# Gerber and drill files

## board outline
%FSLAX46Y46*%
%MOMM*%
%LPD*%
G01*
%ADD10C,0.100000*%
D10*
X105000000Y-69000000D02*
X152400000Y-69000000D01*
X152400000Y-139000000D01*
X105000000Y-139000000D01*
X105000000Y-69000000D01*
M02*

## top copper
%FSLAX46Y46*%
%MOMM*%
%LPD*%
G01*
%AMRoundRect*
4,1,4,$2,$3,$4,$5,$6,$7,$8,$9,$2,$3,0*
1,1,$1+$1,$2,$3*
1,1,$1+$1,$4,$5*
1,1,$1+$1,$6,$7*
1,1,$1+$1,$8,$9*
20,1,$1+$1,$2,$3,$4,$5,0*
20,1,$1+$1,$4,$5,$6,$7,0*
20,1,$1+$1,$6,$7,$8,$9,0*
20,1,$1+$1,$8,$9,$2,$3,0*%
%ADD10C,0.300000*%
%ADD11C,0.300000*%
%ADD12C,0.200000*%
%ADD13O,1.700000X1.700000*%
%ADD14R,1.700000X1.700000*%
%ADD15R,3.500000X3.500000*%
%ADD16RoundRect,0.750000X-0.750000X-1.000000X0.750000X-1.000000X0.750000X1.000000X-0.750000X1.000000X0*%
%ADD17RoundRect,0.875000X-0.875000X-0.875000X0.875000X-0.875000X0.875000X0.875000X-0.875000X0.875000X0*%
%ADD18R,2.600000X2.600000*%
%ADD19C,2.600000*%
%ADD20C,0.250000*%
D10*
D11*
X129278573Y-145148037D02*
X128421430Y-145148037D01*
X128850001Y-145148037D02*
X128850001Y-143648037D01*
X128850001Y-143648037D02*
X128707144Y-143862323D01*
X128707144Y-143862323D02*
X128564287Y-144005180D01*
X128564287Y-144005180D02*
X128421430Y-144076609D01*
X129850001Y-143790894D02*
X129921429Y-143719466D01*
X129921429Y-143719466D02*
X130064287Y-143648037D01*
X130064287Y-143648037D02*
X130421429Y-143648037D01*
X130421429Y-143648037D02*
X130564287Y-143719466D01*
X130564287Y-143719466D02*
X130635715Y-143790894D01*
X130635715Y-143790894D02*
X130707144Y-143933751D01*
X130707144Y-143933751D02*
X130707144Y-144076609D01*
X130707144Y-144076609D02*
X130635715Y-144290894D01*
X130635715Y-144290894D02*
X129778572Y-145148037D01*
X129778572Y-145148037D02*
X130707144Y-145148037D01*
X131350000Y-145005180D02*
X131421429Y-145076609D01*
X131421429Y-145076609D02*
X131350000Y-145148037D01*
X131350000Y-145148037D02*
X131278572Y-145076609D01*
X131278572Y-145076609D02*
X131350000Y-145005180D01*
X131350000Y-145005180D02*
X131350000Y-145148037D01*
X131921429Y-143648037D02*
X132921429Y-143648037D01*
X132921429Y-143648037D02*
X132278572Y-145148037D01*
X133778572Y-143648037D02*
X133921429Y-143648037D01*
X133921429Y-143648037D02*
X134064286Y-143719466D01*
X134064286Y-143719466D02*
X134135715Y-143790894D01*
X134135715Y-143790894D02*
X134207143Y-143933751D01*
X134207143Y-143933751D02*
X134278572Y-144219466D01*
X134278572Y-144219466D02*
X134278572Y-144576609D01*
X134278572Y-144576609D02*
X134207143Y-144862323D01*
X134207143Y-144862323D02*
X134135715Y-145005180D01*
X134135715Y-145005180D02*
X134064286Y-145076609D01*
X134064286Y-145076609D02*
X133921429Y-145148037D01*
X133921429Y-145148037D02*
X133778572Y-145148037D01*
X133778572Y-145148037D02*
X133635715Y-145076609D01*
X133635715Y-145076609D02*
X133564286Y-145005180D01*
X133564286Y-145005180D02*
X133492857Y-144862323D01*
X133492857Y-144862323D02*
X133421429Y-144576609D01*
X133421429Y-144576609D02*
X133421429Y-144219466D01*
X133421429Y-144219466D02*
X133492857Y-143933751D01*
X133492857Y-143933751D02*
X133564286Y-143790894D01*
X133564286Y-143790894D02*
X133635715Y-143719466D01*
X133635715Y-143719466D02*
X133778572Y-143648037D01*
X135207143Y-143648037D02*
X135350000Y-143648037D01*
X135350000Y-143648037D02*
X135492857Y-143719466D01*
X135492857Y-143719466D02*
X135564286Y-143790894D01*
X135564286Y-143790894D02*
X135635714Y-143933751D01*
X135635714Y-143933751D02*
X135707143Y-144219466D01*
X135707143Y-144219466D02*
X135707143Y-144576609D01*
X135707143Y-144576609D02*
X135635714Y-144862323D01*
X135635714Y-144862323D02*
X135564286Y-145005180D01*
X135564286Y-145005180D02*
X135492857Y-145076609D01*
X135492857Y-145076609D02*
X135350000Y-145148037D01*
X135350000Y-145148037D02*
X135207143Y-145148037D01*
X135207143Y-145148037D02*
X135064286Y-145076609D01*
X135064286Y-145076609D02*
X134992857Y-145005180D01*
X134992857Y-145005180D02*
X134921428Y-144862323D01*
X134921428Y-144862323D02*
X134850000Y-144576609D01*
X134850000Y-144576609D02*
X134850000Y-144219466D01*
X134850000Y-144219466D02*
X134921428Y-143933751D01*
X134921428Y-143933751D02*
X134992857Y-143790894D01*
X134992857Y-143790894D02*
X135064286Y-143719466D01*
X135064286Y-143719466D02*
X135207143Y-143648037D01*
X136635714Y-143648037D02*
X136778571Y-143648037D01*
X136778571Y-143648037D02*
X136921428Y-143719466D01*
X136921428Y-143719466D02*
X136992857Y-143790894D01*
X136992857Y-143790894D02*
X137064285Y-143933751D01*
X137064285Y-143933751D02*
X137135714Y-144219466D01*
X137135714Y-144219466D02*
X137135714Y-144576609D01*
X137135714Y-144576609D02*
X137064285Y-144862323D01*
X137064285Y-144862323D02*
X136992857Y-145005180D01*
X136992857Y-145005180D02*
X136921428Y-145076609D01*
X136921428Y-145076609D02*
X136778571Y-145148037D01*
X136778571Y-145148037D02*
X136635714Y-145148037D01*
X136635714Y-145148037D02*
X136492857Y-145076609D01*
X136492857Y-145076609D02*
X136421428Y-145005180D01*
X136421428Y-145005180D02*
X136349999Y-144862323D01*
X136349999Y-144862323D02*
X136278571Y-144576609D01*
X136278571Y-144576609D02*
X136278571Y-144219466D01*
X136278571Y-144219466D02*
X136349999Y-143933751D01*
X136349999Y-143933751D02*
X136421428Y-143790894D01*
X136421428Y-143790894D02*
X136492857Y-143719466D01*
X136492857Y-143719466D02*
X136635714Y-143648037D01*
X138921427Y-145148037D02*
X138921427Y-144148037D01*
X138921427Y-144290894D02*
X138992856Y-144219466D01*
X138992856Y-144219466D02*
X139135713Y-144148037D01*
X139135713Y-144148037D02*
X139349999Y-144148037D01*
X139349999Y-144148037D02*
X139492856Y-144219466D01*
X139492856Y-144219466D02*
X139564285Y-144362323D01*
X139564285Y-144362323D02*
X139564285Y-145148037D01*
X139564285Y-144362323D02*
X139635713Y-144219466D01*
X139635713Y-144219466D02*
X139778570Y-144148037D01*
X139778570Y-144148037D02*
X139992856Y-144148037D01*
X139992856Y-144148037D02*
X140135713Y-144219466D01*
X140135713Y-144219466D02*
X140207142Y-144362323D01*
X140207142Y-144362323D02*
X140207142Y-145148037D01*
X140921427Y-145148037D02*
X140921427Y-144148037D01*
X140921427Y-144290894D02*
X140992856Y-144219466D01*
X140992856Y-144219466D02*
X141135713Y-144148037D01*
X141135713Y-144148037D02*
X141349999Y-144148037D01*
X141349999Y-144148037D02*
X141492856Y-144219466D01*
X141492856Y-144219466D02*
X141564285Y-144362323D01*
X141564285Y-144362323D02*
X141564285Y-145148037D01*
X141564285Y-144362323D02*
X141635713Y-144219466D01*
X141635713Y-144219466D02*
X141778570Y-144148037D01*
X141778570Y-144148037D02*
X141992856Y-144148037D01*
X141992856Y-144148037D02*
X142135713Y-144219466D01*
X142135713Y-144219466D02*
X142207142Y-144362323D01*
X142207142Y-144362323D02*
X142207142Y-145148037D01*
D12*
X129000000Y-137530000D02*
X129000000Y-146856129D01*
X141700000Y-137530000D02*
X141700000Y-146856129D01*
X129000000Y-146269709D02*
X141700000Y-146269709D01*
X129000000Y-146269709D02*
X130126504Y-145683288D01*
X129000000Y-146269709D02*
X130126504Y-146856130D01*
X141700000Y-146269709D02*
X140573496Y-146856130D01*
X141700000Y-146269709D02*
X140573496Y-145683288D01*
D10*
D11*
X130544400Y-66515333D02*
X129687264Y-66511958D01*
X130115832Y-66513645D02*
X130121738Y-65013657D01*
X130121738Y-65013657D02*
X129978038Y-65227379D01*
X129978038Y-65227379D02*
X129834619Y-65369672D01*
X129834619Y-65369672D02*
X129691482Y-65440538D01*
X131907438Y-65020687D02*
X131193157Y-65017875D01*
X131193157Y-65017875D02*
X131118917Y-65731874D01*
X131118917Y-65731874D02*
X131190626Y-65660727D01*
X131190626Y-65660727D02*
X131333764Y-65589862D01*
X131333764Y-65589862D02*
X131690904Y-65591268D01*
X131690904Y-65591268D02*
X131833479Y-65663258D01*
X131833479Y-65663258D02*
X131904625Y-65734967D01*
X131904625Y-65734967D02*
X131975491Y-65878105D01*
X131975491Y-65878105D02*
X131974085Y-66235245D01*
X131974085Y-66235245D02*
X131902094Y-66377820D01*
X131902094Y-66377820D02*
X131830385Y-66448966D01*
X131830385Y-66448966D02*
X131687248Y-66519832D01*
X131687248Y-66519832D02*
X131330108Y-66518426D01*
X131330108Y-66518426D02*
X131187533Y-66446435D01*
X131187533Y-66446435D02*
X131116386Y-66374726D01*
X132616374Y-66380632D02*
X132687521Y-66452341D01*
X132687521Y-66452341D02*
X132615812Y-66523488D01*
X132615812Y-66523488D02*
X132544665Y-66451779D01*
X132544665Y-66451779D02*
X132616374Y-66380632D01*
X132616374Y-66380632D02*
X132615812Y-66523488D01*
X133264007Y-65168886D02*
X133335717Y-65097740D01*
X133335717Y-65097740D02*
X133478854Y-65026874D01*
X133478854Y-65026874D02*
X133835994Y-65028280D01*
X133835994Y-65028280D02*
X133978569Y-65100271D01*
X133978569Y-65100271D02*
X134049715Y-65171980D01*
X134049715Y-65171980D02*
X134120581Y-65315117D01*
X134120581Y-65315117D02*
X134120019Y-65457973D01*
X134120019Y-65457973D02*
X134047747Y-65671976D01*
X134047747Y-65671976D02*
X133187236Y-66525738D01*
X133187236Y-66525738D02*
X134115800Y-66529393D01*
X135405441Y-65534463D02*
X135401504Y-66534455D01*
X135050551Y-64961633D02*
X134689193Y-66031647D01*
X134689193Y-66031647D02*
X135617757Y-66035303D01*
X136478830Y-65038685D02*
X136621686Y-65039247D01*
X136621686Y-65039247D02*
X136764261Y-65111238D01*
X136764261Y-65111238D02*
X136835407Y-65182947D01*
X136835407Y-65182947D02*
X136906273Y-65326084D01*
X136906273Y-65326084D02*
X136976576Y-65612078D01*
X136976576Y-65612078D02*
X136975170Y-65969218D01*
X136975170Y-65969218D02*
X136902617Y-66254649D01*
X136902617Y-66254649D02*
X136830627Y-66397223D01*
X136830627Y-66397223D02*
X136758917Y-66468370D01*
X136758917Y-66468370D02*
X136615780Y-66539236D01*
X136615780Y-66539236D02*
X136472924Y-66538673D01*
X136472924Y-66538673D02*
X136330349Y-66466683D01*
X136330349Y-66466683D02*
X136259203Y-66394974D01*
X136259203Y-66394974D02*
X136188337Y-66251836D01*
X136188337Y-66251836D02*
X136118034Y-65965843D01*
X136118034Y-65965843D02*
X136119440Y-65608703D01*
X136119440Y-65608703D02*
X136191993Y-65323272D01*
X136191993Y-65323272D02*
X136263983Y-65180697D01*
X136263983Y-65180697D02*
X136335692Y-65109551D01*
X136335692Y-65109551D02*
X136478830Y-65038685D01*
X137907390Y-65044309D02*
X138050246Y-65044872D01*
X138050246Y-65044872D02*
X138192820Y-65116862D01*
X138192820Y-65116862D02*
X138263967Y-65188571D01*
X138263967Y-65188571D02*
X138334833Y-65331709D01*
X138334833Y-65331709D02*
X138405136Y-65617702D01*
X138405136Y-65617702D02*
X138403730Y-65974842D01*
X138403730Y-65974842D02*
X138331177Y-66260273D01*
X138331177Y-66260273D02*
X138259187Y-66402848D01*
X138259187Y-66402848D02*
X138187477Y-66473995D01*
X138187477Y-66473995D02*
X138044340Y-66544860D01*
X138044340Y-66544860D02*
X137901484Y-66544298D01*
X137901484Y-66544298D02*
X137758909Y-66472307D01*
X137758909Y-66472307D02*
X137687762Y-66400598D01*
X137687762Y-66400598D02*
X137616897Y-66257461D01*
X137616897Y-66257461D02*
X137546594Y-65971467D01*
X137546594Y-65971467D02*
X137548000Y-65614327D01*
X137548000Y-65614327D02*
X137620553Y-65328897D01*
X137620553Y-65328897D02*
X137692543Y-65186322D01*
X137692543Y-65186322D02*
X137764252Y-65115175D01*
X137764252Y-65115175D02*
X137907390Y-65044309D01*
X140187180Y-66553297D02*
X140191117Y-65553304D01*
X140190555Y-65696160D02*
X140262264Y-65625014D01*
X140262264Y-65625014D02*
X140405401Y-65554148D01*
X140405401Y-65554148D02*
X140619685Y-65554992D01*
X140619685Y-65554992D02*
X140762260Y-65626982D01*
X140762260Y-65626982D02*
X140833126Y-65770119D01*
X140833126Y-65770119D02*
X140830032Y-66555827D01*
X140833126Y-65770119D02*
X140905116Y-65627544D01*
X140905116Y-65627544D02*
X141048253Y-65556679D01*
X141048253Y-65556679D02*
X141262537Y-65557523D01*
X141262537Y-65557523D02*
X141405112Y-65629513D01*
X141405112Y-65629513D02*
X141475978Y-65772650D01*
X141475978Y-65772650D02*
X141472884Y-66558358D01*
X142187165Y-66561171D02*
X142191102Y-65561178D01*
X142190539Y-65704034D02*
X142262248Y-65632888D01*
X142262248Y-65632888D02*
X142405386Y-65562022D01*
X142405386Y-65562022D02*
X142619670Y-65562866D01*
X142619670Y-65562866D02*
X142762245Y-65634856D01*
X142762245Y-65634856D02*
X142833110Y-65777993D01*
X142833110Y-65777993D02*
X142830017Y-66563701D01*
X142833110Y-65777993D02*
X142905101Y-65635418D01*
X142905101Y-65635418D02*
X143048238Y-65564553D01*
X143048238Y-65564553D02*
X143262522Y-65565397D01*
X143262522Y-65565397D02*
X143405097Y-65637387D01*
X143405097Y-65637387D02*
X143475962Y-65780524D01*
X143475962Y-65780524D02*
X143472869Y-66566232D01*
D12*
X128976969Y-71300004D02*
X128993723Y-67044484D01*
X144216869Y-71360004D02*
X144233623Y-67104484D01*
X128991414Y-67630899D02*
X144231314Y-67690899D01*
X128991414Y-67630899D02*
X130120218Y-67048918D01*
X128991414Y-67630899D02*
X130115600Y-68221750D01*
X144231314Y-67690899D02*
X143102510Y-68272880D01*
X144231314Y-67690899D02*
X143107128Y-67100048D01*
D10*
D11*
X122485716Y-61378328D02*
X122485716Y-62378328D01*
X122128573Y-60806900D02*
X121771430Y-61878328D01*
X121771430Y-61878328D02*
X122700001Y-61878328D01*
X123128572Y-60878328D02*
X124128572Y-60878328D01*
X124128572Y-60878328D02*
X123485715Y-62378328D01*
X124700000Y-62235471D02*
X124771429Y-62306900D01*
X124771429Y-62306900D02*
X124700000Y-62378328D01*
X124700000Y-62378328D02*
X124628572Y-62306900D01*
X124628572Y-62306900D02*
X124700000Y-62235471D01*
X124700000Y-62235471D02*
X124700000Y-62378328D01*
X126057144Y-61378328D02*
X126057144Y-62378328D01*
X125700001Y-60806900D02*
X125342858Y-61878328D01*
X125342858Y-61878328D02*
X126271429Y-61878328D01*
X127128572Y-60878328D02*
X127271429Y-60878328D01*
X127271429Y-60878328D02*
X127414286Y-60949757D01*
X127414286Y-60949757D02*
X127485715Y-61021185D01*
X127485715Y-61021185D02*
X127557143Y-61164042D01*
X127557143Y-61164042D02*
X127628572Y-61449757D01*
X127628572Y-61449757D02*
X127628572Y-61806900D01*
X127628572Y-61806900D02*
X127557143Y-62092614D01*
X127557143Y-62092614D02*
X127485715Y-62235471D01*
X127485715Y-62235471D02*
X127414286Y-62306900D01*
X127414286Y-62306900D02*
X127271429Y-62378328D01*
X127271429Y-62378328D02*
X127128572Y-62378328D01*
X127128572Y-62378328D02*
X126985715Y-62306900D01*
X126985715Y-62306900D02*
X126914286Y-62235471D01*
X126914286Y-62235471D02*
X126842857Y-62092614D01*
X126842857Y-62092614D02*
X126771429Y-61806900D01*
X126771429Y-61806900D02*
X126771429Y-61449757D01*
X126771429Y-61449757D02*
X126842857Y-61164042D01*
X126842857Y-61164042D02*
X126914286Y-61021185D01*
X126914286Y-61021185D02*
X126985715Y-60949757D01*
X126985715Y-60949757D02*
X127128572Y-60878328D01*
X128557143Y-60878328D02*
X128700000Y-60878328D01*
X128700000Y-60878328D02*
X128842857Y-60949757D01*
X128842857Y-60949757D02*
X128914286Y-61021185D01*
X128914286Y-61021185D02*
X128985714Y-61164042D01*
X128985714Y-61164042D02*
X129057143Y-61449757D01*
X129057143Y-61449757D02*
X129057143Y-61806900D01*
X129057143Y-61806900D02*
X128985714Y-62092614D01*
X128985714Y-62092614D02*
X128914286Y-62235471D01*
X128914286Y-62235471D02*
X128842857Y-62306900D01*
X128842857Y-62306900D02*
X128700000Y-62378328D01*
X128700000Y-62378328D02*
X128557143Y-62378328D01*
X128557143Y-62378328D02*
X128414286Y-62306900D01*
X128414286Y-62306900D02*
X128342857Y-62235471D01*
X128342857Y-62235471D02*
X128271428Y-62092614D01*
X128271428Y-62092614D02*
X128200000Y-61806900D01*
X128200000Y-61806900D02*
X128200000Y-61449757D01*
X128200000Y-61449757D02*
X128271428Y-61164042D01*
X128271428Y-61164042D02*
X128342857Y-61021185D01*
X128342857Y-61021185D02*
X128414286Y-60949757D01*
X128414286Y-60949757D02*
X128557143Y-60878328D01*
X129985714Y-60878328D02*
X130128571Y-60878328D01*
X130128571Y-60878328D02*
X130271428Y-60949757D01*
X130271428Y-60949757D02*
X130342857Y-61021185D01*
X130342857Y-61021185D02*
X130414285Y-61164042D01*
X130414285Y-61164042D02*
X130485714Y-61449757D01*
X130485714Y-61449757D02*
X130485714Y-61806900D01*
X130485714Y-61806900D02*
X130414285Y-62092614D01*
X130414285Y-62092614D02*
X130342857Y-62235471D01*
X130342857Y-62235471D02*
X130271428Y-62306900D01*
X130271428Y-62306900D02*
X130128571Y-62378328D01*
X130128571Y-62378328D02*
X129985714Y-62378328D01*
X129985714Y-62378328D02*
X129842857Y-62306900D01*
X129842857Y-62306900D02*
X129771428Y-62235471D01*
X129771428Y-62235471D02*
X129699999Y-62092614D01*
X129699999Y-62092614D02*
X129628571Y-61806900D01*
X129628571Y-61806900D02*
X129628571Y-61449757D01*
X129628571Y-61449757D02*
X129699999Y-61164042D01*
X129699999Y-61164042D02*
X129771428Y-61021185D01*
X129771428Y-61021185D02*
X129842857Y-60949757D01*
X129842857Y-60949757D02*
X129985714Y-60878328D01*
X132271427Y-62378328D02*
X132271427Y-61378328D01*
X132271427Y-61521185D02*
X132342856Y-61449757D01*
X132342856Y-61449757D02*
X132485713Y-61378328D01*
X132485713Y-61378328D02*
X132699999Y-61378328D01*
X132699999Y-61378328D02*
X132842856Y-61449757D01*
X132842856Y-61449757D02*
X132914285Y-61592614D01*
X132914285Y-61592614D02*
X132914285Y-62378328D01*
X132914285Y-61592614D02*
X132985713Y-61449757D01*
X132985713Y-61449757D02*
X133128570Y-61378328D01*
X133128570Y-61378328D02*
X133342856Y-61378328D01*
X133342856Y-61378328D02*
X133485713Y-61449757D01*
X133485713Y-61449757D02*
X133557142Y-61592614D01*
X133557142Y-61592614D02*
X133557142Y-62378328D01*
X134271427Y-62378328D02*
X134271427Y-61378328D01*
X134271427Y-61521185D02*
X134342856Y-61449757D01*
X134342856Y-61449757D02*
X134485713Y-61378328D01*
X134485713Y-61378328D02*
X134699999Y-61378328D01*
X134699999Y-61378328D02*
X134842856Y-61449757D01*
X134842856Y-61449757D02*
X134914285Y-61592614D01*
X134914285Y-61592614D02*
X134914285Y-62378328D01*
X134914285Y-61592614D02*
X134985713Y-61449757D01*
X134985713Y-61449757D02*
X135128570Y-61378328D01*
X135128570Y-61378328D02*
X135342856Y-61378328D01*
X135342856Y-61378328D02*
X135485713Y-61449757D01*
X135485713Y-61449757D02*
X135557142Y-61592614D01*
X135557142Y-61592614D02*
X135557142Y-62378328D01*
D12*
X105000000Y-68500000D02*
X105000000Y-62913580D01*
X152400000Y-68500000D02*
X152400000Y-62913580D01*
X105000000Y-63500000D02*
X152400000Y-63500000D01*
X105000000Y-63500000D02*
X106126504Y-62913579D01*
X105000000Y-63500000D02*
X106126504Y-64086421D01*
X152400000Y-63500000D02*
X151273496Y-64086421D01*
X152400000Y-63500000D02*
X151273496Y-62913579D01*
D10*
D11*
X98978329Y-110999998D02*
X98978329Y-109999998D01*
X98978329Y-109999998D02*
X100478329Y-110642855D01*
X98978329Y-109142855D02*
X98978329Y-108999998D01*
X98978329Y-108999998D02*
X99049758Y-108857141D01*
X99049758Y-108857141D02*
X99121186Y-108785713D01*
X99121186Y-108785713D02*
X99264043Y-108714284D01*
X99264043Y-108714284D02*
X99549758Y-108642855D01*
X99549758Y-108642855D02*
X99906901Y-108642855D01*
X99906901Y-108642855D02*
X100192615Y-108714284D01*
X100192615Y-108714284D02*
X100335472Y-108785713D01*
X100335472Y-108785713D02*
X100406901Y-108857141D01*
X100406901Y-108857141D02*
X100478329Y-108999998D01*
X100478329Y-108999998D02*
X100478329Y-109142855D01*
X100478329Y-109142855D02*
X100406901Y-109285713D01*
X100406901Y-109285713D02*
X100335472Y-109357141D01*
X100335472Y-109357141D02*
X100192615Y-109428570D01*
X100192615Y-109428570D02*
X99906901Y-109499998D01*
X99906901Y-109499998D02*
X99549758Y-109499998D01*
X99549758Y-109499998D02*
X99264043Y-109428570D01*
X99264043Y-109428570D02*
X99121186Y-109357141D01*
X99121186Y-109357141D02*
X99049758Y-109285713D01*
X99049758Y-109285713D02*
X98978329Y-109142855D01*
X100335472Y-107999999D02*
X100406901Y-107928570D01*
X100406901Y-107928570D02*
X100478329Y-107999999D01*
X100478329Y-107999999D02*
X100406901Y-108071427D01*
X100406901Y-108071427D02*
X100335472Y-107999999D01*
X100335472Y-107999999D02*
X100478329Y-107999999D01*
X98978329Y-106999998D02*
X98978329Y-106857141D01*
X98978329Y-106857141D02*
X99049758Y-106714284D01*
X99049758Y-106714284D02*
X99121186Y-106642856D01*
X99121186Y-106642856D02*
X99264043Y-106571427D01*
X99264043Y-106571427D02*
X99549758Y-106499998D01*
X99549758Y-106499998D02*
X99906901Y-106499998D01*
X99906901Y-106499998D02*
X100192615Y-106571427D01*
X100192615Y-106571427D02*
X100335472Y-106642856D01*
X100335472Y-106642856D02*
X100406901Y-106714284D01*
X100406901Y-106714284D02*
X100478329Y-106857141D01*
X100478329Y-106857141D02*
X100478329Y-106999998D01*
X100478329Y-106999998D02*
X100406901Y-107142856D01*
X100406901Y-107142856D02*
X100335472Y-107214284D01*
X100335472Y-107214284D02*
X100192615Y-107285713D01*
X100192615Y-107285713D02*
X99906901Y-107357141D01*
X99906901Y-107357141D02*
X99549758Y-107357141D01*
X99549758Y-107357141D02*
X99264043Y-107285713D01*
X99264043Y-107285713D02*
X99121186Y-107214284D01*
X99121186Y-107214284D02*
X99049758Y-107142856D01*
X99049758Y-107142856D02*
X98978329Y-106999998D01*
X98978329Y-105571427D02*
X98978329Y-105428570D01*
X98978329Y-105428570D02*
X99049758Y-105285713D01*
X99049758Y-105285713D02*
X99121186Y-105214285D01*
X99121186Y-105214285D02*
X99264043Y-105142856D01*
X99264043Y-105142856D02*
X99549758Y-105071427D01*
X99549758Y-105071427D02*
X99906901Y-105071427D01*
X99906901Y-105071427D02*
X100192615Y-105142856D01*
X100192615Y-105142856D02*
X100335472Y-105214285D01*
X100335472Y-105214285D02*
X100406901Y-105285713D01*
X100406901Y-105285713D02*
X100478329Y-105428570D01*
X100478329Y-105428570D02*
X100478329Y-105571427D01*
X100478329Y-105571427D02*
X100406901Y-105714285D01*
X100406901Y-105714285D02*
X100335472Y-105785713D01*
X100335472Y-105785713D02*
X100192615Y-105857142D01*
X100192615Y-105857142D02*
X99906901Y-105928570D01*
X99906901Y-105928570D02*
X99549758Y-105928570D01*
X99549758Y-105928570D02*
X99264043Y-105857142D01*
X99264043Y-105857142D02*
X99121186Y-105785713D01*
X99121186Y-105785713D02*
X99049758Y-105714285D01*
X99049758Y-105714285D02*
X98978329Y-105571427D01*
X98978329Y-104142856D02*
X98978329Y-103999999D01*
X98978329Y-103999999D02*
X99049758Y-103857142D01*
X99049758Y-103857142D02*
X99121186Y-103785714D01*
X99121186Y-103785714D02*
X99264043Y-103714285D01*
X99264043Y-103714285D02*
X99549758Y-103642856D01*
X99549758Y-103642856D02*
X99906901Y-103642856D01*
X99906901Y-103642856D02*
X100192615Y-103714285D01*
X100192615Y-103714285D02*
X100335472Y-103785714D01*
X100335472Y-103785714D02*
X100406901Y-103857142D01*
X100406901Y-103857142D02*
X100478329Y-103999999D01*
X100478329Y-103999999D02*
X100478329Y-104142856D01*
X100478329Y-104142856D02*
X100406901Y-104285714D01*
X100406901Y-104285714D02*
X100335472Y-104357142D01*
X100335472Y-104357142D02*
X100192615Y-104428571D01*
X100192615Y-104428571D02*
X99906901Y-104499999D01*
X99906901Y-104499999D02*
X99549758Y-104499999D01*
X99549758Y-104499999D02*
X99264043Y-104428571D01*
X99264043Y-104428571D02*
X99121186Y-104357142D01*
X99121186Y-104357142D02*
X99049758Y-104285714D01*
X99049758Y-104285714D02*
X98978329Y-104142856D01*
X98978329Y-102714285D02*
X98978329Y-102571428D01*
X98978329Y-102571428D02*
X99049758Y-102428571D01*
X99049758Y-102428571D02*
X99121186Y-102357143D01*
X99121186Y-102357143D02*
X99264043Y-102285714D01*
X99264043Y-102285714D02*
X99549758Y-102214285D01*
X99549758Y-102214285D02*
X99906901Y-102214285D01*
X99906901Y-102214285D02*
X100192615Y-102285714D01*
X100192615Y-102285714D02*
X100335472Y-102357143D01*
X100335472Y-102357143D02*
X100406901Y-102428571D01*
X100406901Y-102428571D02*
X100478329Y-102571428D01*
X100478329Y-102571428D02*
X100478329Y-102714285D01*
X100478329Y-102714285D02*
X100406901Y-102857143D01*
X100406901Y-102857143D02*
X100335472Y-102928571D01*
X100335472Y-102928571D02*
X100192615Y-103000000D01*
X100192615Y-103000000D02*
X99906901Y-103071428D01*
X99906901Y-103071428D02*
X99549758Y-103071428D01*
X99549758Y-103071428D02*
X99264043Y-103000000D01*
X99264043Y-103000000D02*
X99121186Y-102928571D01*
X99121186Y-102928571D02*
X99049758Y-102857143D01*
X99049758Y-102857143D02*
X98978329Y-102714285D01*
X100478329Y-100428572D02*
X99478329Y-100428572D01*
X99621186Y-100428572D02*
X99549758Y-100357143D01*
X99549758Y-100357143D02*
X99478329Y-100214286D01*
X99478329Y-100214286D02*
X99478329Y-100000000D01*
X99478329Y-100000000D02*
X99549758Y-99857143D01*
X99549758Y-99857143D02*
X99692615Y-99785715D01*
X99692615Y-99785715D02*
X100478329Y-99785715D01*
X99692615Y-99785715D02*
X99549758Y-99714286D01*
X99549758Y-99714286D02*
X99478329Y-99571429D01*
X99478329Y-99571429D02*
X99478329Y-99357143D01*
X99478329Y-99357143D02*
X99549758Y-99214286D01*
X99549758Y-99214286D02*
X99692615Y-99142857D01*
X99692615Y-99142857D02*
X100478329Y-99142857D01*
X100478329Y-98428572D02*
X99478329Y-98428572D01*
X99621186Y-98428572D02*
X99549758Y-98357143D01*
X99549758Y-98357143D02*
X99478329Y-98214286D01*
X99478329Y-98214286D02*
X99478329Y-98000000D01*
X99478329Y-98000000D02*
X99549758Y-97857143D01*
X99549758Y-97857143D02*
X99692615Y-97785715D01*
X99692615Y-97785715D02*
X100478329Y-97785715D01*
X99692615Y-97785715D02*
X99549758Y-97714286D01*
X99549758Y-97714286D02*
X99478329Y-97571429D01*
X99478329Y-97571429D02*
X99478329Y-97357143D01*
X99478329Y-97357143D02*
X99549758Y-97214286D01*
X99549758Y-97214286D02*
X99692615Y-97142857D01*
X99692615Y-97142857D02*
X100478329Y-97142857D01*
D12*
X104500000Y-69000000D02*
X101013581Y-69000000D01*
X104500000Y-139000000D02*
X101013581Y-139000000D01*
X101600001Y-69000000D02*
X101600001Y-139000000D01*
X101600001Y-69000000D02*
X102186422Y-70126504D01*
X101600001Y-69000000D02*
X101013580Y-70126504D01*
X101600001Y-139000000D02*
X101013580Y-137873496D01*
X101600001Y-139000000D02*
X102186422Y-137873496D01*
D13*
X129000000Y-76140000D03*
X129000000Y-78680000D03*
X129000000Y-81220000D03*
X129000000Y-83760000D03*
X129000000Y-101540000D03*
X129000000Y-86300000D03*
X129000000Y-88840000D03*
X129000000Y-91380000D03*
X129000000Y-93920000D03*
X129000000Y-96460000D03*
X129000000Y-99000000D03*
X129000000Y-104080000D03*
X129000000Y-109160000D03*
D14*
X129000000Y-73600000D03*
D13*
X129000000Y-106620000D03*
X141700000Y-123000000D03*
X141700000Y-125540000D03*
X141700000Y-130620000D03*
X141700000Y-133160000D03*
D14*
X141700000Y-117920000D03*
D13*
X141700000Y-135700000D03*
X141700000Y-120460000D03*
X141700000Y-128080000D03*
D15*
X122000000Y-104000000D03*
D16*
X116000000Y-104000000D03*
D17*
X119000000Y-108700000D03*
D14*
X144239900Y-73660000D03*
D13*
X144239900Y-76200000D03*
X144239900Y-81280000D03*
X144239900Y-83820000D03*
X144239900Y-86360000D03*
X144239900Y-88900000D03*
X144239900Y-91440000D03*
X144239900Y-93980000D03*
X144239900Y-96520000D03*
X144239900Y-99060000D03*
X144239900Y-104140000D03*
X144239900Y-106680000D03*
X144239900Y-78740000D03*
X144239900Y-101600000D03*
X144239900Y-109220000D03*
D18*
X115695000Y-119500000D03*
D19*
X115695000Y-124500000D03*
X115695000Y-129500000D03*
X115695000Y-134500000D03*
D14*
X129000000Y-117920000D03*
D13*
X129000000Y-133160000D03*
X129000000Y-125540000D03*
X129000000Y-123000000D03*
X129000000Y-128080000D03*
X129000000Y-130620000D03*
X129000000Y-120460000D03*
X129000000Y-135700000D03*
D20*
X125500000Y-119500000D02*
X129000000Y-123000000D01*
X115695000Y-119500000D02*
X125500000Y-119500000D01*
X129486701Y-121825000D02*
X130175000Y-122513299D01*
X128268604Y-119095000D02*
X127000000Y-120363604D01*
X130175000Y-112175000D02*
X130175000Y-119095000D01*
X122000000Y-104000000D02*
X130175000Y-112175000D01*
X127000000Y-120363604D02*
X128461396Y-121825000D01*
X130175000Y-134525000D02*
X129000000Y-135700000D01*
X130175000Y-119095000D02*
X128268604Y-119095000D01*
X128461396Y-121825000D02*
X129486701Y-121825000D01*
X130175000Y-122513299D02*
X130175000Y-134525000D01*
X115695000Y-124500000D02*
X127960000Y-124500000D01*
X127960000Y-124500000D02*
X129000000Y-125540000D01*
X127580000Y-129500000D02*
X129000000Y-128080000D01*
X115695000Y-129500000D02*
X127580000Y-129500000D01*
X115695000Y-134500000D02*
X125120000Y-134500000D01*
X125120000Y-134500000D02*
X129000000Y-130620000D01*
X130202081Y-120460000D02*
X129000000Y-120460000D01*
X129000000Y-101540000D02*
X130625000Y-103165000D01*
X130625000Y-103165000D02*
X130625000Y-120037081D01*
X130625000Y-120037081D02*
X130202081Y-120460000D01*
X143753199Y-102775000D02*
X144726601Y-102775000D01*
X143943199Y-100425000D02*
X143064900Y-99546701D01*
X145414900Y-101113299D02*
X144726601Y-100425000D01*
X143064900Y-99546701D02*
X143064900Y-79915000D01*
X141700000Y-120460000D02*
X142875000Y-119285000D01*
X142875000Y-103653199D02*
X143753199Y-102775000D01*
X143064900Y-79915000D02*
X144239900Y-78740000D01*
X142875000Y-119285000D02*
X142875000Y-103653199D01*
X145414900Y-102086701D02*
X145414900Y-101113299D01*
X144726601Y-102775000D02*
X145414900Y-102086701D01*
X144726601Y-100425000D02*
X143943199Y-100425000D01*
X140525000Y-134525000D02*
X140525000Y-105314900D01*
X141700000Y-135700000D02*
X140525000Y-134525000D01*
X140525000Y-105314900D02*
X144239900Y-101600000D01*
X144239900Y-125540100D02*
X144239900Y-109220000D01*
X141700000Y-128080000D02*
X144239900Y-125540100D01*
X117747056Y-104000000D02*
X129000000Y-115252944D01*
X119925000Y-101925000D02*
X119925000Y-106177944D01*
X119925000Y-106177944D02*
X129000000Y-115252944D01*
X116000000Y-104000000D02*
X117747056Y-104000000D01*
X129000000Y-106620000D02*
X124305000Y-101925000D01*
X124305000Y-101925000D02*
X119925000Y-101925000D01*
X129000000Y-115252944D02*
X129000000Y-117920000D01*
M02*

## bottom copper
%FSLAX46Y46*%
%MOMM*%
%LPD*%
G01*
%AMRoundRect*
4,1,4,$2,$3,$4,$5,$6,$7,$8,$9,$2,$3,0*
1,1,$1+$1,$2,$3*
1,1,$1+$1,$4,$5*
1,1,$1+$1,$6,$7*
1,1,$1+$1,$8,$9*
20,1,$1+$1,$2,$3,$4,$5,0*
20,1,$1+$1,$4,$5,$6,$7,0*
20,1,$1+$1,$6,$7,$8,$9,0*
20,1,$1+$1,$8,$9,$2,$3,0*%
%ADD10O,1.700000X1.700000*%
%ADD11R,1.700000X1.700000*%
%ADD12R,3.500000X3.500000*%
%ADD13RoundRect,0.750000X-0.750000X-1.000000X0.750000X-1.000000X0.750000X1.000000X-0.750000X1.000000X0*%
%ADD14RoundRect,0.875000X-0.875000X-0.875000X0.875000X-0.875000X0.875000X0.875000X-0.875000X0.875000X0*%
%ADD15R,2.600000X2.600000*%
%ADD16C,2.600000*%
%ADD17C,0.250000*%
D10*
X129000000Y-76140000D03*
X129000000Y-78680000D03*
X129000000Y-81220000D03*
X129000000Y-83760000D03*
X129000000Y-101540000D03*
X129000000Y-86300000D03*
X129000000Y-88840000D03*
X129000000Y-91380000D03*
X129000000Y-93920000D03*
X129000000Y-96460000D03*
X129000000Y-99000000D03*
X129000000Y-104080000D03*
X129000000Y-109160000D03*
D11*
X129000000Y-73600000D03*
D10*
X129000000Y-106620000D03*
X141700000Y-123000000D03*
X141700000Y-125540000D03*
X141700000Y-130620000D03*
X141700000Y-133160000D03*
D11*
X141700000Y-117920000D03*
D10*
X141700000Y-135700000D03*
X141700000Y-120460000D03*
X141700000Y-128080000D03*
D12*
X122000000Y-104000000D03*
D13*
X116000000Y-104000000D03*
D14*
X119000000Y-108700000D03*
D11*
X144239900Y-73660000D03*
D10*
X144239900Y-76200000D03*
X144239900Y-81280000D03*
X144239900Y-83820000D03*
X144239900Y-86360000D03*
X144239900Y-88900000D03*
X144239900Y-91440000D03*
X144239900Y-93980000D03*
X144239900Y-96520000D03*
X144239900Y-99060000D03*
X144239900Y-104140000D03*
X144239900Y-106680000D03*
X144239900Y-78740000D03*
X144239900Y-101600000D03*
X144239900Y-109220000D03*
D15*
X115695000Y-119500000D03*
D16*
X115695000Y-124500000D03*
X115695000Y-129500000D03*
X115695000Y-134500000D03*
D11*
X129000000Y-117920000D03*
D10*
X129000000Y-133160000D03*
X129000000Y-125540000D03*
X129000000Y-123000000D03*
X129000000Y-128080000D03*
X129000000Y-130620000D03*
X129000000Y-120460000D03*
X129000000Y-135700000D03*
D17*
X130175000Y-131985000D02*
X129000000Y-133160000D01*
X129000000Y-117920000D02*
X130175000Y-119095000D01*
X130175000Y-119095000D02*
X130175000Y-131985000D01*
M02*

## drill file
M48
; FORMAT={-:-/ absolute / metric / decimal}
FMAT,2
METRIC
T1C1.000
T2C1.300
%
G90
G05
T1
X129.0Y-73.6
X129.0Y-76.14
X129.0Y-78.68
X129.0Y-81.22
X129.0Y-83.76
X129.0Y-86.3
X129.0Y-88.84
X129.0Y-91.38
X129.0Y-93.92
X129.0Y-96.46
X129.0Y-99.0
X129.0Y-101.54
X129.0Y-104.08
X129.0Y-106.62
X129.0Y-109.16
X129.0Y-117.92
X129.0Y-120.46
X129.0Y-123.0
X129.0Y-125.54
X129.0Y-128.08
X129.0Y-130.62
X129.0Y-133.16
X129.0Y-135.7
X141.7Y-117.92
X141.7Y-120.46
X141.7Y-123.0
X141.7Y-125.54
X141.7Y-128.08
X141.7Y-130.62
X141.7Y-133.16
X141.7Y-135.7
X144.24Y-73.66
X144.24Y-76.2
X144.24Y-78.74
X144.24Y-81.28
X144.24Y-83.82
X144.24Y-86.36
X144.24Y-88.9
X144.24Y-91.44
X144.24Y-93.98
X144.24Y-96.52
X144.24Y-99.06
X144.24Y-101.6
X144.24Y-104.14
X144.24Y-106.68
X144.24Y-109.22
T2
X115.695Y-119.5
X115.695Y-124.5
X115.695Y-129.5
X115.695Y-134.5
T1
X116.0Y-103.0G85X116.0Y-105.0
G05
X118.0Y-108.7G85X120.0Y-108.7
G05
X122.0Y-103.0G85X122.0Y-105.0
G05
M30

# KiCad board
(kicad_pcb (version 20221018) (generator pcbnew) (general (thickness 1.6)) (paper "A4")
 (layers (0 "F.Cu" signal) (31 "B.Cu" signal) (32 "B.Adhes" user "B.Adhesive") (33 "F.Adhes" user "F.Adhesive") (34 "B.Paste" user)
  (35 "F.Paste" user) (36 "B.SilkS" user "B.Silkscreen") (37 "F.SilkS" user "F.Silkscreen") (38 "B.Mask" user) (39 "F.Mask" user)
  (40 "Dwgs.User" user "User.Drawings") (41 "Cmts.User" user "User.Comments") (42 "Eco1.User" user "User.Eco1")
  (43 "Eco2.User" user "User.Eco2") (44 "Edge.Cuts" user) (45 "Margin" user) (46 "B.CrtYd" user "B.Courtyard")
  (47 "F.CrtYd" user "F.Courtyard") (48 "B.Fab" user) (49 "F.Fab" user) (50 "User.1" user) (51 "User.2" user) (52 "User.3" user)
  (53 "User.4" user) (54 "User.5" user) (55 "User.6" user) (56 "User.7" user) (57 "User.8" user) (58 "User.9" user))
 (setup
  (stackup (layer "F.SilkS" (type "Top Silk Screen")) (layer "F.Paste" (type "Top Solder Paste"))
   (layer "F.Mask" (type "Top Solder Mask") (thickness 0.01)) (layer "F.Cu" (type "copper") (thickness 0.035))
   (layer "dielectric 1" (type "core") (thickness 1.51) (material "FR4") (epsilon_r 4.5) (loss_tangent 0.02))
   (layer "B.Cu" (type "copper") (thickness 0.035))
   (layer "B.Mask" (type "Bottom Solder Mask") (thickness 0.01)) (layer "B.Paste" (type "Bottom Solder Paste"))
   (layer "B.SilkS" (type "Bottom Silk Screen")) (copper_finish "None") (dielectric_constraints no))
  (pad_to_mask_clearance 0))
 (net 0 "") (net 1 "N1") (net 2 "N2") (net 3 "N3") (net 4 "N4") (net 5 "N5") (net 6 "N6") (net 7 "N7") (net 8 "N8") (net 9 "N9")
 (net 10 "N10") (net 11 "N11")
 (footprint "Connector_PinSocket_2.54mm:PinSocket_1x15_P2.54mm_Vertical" (layer "F.Cu") (at 129 73.6)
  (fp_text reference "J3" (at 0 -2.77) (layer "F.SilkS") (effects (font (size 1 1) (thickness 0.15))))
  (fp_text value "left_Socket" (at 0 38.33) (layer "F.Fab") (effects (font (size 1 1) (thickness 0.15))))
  (pad "2" thru_hole oval (at 0 2.54) (size 1.7 1.7) (drill 1) (layers "*.Cu" "*.Mask"))
  (pad "3" thru_hole oval (at 0 5.08) (size 1.7 1.7) (drill 1) (layers "*.Cu" "*.Mask"))
  (pad "4" thru_hole oval (at 0 7.62) (size 1.7 1.7) (drill 1) (layers "*.Cu" "*.Mask"))
  (pad "5" thru_hole oval (at 0 10.16) (size 1.7 1.7) (drill 1) (layers "*.Cu" "*.Mask"))
  (pad "5V" thru_hole oval (at 0 27.94) (size 1.7 1.7) (drill 1) (layers "*.Cu" "*.Mask") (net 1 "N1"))
  (pad "6" thru_hole oval (at 0 12.7) (size 1.7 1.7) (drill 1) (layers "*.Cu" "*.Mask"))
  (pad "7" thru_hole oval (at 0 15.24) (size 1.7 1.7) (drill 1) (layers "*.Cu" "*.Mask"))
  (pad "8" thru_hole oval (at 0 17.78) (size 1.7 1.7) (drill 1) (layers "*.Cu" "*.Mask"))
  (pad "9" thru_hole oval (at 0 20.32) (size 1.7 1.7) (drill 1) (layers "*.Cu" "*.Mask"))
  (pad "10" thru_hole oval (at 0 22.86) (size 1.7 1.7) (drill 1) (layers "*.Cu" "*.Mask"))
  (pad "11" thru_hole oval (at 0 25.4) (size 1.7 1.7) (drill 1) (layers "*.Cu" "*.Mask"))
  (pad "13" thru_hole oval (at 0 30.48) (size 1.7 1.7) (drill 1) (layers "*.Cu" "*.Mask"))
  (pad "15" thru_hole oval (at 0 35.56) (size 1.7 1.7) (drill 1) (layers "*.Cu" "*.Mask"))
  (pad "D12" thru_hole rect (at 0 0) (size 1.7 1.7) (drill 1) (layers "*.Cu" "*.Mask"))
  (pad "GND" thru_hole oval (at 0 33.02) (size 1.7 1.7) (drill 1) (layers "*.Cu" "*.Mask") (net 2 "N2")))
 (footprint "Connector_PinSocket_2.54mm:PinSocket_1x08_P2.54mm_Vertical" (layer "F.Cu") (at 141.7 117.92)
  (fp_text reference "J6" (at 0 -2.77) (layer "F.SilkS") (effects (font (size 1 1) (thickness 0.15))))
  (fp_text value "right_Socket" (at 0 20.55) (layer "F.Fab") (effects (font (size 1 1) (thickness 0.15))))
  (pad "3" thru_hole oval (at 0 5.08) (size 1.7 1.7) (drill 1) (layers "*.Cu" "*.Mask"))
  (pad "4" thru_hole oval (at 0 7.62) (size 1.7 1.7) (drill 1) (layers "*.Cu" "*.Mask"))
  (pad "6" thru_hole oval (at 0 12.7) (size 1.7 1.7) (drill 1) (layers "*.Cu" "*.Mask"))
  (pad "7" thru_hole oval (at 0 15.24) (size 1.7 1.7) (drill 1) (layers "*.Cu" "*.Mask"))
  (pad "Dir" thru_hole rect (at 0 0) (size 1.7 1.7) (drill 1) (layers "*.Cu" "*.Mask") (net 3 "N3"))
  (pad "EN" thru_hole oval (at 0 17.78) (size 1.7 1.7) (drill 1) (layers "*.Cu" "*.Mask") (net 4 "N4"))
  (pad "Step" thru_hole oval (at 0 2.54) (size 1.7 1.7) (drill 1) (layers "*.Cu" "*.Mask") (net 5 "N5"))
  (pad "UART" thru_hole oval (at 0 10.16) (size 1.7 1.7) (drill 1) (layers "*.Cu" "*.Mask") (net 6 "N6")))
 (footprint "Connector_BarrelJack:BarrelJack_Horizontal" (layer "F.Cu") (at 122 104)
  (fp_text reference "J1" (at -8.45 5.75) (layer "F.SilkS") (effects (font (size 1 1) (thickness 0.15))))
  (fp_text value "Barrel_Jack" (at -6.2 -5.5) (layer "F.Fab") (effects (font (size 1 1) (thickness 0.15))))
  (pad "1" thru_hole rect (at 0 0) (size 3.5 3.5) (drill oval 1 3) (layers "*.Cu" "*.Mask") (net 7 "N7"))
  (pad "2" thru_hole roundrect (at -6 0) (size 3 3.5) (drill oval 1 3) (layers "*.Cu" "*.Mask") (roundrect_rratio 0.25) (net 2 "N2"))
  (pad "3" thru_hole roundrect (at -3 4.7) (size 3.5 3.5) (drill oval 3 1) (layers "*.Cu" "*.Mask") (roundrect_rratio 0.25)))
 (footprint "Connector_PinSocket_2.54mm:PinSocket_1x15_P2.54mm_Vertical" (layer "F.Cu") (at 144.2399 73.66)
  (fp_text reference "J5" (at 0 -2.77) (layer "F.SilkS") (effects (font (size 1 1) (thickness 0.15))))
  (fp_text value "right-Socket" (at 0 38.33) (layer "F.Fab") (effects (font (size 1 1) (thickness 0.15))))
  (pad "1" thru_hole rect (at 0 0) (size 1.7 1.7) (drill 1) (layers "*.Cu" "*.Mask"))
  (pad "2" thru_hole oval (at 0 2.54) (size 1.7 1.7) (drill 1) (layers "*.Cu" "*.Mask"))
  (pad "4" thru_hole oval (at 0 7.62) (size 1.7 1.7) (drill 1) (layers "*.Cu" "*.Mask"))
  (pad "5" thru_hole oval (at 0 10.16) (size 1.7 1.7) (drill 1) (layers "*.Cu" "*.Mask"))
  (pad "6" thru_hole oval (at 0 12.7) (size 1.7 1.7) (drill 1) (layers "*.Cu" "*.Mask"))
  (pad "7" thru_hole oval (at 0 15.24) (size 1.7 1.7) (drill 1) (layers "*.Cu" "*.Mask"))
  (pad "8" thru_hole oval (at 0 17.78) (size 1.7 1.7) (drill 1) (layers "*.Cu" "*.Mask"))
  (pad "9" thru_hole oval (at 0 20.32) (size 1.7 1.7) (drill 1) (layers "*.Cu" "*.Mask"))
  (pad "10" thru_hole oval (at 0 22.86) (size 1.7 1.7) (drill 1) (layers "*.Cu" "*.Mask"))
  (pad "11" thru_hole oval (at 0 25.4) (size 1.7 1.7) (drill 1) (layers "*.Cu" "*.Mask"))
  (pad "13" thru_hole oval (at 0 30.48) (size 1.7 1.7) (drill 1) (layers "*.Cu" "*.Mask"))
  (pad "14" thru_hole oval (at 0 33.02) (size 1.7 1.7) (drill 1) (layers "*.Cu" "*.Mask"))
  (pad "D10" thru_hole oval (at 0 5.08) (size 1.7 1.7) (drill 1) (layers "*.Cu" "*.Mask") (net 5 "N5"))
  (pad "GND" thru_hole oval (at 0 27.94) (size 1.7 1.7) (drill 1) (layers "*.Cu" "*.Mask") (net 4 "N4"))
  (pad "TX1" thru_hole oval (at 0 35.56) (size 1.7 1.7) (drill 1) (layers "*.Cu" "*.Mask") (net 6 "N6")))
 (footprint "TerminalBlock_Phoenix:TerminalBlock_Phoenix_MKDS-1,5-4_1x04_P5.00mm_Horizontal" (layer "F.Cu") (at 115.695 119.5 -90)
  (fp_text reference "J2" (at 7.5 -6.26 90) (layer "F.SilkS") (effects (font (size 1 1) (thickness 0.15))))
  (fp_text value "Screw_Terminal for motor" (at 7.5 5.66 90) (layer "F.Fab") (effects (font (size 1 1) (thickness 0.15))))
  (pad "1" thru_hole rect (at 0 0 270) (size 2.6 2.6) (drill 1.3) (layers "*.Cu" "*.Mask") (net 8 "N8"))
  (pad "2" thru_hole circle (at 5 0 270) (size 2.6 2.6) (drill 1.3) (layers "*.Cu" "*.Mask") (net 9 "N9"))
  (pad "3" thru_hole circle (at 10 0 270) (size 2.6 2.6) (drill 1.3) (layers "*.Cu" "*.Mask") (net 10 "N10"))
  (pad "4" thru_hole circle (at 15 0 270) (size 2.6 2.6) (drill 1.3) (layers "*.Cu" "*.Mask") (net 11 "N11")))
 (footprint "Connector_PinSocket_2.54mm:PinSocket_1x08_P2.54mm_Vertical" (layer "F.Cu") (at 129 117.92)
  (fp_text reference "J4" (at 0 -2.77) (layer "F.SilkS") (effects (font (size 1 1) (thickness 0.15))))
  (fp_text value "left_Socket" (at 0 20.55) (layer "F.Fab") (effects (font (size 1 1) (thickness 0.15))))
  (pad "GND" thru_hole rect (at 0 0) (size 1.7 1.7) (drill 1) (layers "*.Cu" "*.Mask") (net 2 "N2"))
  (pad "GND" thru_hole oval (at 0 15.24) (size 1.7 1.7) (drill 1) (layers "*.Cu" "*.Mask") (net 2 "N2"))
  (pad "M1A" thru_hole oval (at 0 7.62) (size 1.7 1.7) (drill 1) (layers "*.Cu" "*.Mask") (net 9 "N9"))
  (pad "M1B" thru_hole oval (at 0 5.08) (size 1.7 1.7) (drill 1) (layers "*.Cu" "*.Mask") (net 8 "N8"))
  (pad "M2A" thru_hole oval (at 0 10.16) (size 1.7 1.7) (drill 1) (layers "*.Cu" "*.Mask") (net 10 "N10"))
  (pad "M2B" thru_hole oval (at 0 12.7) (size 1.7 1.7) (drill 1) (layers "*.Cu" "*.Mask") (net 11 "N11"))
  (pad "VIO" thru_hole oval (at 0 2.54) (size 1.7 1.7) (drill 1) (layers "*.Cu" "*.Mask") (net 1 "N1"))
  (pad "VM" thru_hole oval (at 0 17.78) (size 1.7 1.7) (drill 1) (layers "*.Cu" "*.Mask") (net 7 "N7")))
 (gr_rect (start 105 69) (end 152.4 139) (stroke (width 0.1) (type default)) (fill none) (layer "Edge.Cuts"))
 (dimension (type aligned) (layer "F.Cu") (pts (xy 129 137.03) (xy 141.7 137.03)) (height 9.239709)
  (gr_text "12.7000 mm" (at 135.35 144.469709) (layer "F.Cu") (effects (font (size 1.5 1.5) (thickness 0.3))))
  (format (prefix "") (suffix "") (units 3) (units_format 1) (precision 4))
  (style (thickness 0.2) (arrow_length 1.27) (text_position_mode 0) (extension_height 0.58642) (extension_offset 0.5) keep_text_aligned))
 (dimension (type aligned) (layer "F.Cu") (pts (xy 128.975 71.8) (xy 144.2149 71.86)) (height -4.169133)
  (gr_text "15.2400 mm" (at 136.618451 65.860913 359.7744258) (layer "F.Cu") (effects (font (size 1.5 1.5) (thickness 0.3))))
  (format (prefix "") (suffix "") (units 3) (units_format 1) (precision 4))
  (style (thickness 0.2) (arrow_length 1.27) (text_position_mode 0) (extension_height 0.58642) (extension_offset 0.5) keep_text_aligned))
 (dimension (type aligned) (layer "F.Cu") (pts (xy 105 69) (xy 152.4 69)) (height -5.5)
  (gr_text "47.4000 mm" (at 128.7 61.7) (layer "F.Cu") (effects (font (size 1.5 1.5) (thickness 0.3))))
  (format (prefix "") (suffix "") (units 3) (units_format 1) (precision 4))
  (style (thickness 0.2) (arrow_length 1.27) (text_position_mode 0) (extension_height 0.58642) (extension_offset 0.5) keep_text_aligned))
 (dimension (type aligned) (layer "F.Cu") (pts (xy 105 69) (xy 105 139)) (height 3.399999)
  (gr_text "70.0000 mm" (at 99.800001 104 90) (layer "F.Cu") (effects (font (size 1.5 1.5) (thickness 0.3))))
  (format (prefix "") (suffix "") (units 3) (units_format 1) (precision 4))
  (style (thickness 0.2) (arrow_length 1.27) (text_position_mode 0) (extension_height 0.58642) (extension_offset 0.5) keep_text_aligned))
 (segment (start 125.5 119.5) (end 129 123) (width 0.25) (layer "F.Cu") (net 8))
 (segment (start 115.695 119.5) (end 125.5 119.5) (width 0.25) (layer "F.Cu") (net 8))
 (segment (start 129.486701 121.825) (end 130.175 122.513299) (width 0.25) (layer "F.Cu") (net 7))
 (segment (start 128.268604 119.095) (end 127 120.363604) (width 0.25) (layer "F.Cu") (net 7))
 (segment (start 130.175 112.175) (end 130.175 119.095) (width 0.25) (layer "F.Cu") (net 7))
 (segment (start 122 104) (end 130.175 112.175) (width 0.25) (layer "F.Cu") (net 7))
 (segment (start 127 120.363604) (end 128.461396 121.825) (width 0.25) (layer "F.Cu") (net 7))
 (segment (start 130.175 134.525) (end 129 135.7) (width 0.25) (layer "F.Cu") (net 7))
 (segment (start 130.175 119.095) (end 128.268604 119.095) (width 0.25) (layer "F.Cu") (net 7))
 (segment (start 128.461396 121.825) (end 129.486701 121.825) (width 0.25) (layer "F.Cu") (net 7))
 (segment (start 130.175 122.513299) (end 130.175 134.525) (width 0.25) (layer "F.Cu") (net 7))
 (segment (start 115.695 124.5) (end 127.96 124.5) (width 0.25) (layer "F.Cu") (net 9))
 (segment (start 127.96 124.5) (end 129 125.54) (width 0.25) (layer "F.Cu") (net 9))
 (segment (start 127.58 129.5) (end 129 128.08) (width 0.25) (layer "F.Cu") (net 10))
 (segment (start 115.695 129.5) (end 127.58 129.5) (width 0.25) (layer "F.Cu") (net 10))
 (segment (start 115.695 134.5) (end 125.12 134.5) (width 0.25) (layer "F.Cu") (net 11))
 (segment (start 125.12 134.5) (end 129 130.62) (width 0.25) (layer "F.Cu") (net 11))
 (segment (start 130.202081 120.46) (end 129 120.46) (width 0.25) (layer "F.Cu") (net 1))
 (segment (start 129 101.54) (end 130.625 103.165) (width 0.25) (layer "F.Cu") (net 1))
 (segment (start 130.625 103.165) (end 130.625 120.037081) (width 0.25) (layer "F.Cu") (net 1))
 (segment (start 130.625 120.037081) (end 130.202081 120.46) (width 0.25) (layer "F.Cu") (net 1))
 (segment (start 143.753199 102.775) (end 144.726601 102.775) (width 0.25) (layer "F.Cu") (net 5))
 (segment (start 143.943199 100.425) (end 143.0649 99.546701) (width 0.25) (layer "F.Cu") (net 5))
 (segment (start 145.4149 101.113299) (end 144.726601 100.425) (width 0.25) (layer "F.Cu") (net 5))
 (segment (start 143.0649 99.546701) (end 143.0649 79.915) (width 0.25) (layer "F.Cu") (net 5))
 (segment (start 141.7 120.46) (end 142.875 119.285) (width 0.25) (layer "F.Cu") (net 5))
 (segment (start 142.875 103.653199) (end 143.753199 102.775) (width 0.25) (layer "F.Cu") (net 5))
 (segment (start 143.0649 79.915) (end 144.2399 78.74) (width 0.25) (layer "F.Cu") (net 5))
 (segment (start 142.875 119.285) (end 142.875 103.653199) (width 0.25) (layer "F.Cu") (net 5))
 (segment (start 145.4149 102.086701) (end 145.4149 101.113299) (width 0.25) (layer "F.Cu") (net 5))
 (segment (start 144.726601 102.775) (end 145.4149 102.086701) (width 0.25) (layer "F.Cu") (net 5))
 (segment (start 144.726601 100.425) (end 143.943199 100.425) (width 0.25) (layer "F.Cu") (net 5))
 (segment (start 140.525 134.525) (end 140.525 105.3149) (width 0.25) (layer "F.Cu") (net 4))
 (segment (start 141.7 135.7) (end 140.525 134.525) (width 0.25) (layer "F.Cu") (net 4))
 (segment (start 140.525 105.3149) (end 144.2399 101.6) (width 0.25) (layer "F.Cu") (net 4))
 (segment (start 144.2399 125.5401) (end 144.2399 109.22) (width 0.25) (layer "F.Cu") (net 6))
 (segment (start 141.7 128.08) (end 144.2399 125.5401) (width 0.25) (layer "F.Cu") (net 6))
 (segment (start 117.747056 104) (end 129 115.252944) (width 0.25) (layer "F.Cu") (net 2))
 (segment (start 119.925 101.925) (end 119.925 106.177944) (width 0.25) (layer "F.Cu") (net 2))
 (segment (start 119.925 106.177944) (end 129 115.252944) (width 0.25) (layer "F.Cu") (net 2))
 (segment (start 116 104) (end 117.747056 104) (width 0.25) (layer "F.Cu") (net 2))
 (segment (start 129 106.62) (end 124.305 101.925) (width 0.25) (layer "F.Cu") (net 2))
 (segment (start 124.305 101.925) (end 119.925 101.925) (width 0.25) (layer "F.Cu") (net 2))
 (segment (start 129 115.252944) (end 129 117.92) (width 0.25) (layer "F.Cu") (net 2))
 (segment (start 130.175 131.985) (end 129 133.16) (width 0.25) (layer "B.Cu") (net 2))
 (segment (start 129 117.92) (end 130.175 119.095) (width 0.25) (layer "B.Cu") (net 2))
 (segment (start 130.175 119.095) (end 130.175 131.985) (width 0.25) (layer "B.Cu") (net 2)))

